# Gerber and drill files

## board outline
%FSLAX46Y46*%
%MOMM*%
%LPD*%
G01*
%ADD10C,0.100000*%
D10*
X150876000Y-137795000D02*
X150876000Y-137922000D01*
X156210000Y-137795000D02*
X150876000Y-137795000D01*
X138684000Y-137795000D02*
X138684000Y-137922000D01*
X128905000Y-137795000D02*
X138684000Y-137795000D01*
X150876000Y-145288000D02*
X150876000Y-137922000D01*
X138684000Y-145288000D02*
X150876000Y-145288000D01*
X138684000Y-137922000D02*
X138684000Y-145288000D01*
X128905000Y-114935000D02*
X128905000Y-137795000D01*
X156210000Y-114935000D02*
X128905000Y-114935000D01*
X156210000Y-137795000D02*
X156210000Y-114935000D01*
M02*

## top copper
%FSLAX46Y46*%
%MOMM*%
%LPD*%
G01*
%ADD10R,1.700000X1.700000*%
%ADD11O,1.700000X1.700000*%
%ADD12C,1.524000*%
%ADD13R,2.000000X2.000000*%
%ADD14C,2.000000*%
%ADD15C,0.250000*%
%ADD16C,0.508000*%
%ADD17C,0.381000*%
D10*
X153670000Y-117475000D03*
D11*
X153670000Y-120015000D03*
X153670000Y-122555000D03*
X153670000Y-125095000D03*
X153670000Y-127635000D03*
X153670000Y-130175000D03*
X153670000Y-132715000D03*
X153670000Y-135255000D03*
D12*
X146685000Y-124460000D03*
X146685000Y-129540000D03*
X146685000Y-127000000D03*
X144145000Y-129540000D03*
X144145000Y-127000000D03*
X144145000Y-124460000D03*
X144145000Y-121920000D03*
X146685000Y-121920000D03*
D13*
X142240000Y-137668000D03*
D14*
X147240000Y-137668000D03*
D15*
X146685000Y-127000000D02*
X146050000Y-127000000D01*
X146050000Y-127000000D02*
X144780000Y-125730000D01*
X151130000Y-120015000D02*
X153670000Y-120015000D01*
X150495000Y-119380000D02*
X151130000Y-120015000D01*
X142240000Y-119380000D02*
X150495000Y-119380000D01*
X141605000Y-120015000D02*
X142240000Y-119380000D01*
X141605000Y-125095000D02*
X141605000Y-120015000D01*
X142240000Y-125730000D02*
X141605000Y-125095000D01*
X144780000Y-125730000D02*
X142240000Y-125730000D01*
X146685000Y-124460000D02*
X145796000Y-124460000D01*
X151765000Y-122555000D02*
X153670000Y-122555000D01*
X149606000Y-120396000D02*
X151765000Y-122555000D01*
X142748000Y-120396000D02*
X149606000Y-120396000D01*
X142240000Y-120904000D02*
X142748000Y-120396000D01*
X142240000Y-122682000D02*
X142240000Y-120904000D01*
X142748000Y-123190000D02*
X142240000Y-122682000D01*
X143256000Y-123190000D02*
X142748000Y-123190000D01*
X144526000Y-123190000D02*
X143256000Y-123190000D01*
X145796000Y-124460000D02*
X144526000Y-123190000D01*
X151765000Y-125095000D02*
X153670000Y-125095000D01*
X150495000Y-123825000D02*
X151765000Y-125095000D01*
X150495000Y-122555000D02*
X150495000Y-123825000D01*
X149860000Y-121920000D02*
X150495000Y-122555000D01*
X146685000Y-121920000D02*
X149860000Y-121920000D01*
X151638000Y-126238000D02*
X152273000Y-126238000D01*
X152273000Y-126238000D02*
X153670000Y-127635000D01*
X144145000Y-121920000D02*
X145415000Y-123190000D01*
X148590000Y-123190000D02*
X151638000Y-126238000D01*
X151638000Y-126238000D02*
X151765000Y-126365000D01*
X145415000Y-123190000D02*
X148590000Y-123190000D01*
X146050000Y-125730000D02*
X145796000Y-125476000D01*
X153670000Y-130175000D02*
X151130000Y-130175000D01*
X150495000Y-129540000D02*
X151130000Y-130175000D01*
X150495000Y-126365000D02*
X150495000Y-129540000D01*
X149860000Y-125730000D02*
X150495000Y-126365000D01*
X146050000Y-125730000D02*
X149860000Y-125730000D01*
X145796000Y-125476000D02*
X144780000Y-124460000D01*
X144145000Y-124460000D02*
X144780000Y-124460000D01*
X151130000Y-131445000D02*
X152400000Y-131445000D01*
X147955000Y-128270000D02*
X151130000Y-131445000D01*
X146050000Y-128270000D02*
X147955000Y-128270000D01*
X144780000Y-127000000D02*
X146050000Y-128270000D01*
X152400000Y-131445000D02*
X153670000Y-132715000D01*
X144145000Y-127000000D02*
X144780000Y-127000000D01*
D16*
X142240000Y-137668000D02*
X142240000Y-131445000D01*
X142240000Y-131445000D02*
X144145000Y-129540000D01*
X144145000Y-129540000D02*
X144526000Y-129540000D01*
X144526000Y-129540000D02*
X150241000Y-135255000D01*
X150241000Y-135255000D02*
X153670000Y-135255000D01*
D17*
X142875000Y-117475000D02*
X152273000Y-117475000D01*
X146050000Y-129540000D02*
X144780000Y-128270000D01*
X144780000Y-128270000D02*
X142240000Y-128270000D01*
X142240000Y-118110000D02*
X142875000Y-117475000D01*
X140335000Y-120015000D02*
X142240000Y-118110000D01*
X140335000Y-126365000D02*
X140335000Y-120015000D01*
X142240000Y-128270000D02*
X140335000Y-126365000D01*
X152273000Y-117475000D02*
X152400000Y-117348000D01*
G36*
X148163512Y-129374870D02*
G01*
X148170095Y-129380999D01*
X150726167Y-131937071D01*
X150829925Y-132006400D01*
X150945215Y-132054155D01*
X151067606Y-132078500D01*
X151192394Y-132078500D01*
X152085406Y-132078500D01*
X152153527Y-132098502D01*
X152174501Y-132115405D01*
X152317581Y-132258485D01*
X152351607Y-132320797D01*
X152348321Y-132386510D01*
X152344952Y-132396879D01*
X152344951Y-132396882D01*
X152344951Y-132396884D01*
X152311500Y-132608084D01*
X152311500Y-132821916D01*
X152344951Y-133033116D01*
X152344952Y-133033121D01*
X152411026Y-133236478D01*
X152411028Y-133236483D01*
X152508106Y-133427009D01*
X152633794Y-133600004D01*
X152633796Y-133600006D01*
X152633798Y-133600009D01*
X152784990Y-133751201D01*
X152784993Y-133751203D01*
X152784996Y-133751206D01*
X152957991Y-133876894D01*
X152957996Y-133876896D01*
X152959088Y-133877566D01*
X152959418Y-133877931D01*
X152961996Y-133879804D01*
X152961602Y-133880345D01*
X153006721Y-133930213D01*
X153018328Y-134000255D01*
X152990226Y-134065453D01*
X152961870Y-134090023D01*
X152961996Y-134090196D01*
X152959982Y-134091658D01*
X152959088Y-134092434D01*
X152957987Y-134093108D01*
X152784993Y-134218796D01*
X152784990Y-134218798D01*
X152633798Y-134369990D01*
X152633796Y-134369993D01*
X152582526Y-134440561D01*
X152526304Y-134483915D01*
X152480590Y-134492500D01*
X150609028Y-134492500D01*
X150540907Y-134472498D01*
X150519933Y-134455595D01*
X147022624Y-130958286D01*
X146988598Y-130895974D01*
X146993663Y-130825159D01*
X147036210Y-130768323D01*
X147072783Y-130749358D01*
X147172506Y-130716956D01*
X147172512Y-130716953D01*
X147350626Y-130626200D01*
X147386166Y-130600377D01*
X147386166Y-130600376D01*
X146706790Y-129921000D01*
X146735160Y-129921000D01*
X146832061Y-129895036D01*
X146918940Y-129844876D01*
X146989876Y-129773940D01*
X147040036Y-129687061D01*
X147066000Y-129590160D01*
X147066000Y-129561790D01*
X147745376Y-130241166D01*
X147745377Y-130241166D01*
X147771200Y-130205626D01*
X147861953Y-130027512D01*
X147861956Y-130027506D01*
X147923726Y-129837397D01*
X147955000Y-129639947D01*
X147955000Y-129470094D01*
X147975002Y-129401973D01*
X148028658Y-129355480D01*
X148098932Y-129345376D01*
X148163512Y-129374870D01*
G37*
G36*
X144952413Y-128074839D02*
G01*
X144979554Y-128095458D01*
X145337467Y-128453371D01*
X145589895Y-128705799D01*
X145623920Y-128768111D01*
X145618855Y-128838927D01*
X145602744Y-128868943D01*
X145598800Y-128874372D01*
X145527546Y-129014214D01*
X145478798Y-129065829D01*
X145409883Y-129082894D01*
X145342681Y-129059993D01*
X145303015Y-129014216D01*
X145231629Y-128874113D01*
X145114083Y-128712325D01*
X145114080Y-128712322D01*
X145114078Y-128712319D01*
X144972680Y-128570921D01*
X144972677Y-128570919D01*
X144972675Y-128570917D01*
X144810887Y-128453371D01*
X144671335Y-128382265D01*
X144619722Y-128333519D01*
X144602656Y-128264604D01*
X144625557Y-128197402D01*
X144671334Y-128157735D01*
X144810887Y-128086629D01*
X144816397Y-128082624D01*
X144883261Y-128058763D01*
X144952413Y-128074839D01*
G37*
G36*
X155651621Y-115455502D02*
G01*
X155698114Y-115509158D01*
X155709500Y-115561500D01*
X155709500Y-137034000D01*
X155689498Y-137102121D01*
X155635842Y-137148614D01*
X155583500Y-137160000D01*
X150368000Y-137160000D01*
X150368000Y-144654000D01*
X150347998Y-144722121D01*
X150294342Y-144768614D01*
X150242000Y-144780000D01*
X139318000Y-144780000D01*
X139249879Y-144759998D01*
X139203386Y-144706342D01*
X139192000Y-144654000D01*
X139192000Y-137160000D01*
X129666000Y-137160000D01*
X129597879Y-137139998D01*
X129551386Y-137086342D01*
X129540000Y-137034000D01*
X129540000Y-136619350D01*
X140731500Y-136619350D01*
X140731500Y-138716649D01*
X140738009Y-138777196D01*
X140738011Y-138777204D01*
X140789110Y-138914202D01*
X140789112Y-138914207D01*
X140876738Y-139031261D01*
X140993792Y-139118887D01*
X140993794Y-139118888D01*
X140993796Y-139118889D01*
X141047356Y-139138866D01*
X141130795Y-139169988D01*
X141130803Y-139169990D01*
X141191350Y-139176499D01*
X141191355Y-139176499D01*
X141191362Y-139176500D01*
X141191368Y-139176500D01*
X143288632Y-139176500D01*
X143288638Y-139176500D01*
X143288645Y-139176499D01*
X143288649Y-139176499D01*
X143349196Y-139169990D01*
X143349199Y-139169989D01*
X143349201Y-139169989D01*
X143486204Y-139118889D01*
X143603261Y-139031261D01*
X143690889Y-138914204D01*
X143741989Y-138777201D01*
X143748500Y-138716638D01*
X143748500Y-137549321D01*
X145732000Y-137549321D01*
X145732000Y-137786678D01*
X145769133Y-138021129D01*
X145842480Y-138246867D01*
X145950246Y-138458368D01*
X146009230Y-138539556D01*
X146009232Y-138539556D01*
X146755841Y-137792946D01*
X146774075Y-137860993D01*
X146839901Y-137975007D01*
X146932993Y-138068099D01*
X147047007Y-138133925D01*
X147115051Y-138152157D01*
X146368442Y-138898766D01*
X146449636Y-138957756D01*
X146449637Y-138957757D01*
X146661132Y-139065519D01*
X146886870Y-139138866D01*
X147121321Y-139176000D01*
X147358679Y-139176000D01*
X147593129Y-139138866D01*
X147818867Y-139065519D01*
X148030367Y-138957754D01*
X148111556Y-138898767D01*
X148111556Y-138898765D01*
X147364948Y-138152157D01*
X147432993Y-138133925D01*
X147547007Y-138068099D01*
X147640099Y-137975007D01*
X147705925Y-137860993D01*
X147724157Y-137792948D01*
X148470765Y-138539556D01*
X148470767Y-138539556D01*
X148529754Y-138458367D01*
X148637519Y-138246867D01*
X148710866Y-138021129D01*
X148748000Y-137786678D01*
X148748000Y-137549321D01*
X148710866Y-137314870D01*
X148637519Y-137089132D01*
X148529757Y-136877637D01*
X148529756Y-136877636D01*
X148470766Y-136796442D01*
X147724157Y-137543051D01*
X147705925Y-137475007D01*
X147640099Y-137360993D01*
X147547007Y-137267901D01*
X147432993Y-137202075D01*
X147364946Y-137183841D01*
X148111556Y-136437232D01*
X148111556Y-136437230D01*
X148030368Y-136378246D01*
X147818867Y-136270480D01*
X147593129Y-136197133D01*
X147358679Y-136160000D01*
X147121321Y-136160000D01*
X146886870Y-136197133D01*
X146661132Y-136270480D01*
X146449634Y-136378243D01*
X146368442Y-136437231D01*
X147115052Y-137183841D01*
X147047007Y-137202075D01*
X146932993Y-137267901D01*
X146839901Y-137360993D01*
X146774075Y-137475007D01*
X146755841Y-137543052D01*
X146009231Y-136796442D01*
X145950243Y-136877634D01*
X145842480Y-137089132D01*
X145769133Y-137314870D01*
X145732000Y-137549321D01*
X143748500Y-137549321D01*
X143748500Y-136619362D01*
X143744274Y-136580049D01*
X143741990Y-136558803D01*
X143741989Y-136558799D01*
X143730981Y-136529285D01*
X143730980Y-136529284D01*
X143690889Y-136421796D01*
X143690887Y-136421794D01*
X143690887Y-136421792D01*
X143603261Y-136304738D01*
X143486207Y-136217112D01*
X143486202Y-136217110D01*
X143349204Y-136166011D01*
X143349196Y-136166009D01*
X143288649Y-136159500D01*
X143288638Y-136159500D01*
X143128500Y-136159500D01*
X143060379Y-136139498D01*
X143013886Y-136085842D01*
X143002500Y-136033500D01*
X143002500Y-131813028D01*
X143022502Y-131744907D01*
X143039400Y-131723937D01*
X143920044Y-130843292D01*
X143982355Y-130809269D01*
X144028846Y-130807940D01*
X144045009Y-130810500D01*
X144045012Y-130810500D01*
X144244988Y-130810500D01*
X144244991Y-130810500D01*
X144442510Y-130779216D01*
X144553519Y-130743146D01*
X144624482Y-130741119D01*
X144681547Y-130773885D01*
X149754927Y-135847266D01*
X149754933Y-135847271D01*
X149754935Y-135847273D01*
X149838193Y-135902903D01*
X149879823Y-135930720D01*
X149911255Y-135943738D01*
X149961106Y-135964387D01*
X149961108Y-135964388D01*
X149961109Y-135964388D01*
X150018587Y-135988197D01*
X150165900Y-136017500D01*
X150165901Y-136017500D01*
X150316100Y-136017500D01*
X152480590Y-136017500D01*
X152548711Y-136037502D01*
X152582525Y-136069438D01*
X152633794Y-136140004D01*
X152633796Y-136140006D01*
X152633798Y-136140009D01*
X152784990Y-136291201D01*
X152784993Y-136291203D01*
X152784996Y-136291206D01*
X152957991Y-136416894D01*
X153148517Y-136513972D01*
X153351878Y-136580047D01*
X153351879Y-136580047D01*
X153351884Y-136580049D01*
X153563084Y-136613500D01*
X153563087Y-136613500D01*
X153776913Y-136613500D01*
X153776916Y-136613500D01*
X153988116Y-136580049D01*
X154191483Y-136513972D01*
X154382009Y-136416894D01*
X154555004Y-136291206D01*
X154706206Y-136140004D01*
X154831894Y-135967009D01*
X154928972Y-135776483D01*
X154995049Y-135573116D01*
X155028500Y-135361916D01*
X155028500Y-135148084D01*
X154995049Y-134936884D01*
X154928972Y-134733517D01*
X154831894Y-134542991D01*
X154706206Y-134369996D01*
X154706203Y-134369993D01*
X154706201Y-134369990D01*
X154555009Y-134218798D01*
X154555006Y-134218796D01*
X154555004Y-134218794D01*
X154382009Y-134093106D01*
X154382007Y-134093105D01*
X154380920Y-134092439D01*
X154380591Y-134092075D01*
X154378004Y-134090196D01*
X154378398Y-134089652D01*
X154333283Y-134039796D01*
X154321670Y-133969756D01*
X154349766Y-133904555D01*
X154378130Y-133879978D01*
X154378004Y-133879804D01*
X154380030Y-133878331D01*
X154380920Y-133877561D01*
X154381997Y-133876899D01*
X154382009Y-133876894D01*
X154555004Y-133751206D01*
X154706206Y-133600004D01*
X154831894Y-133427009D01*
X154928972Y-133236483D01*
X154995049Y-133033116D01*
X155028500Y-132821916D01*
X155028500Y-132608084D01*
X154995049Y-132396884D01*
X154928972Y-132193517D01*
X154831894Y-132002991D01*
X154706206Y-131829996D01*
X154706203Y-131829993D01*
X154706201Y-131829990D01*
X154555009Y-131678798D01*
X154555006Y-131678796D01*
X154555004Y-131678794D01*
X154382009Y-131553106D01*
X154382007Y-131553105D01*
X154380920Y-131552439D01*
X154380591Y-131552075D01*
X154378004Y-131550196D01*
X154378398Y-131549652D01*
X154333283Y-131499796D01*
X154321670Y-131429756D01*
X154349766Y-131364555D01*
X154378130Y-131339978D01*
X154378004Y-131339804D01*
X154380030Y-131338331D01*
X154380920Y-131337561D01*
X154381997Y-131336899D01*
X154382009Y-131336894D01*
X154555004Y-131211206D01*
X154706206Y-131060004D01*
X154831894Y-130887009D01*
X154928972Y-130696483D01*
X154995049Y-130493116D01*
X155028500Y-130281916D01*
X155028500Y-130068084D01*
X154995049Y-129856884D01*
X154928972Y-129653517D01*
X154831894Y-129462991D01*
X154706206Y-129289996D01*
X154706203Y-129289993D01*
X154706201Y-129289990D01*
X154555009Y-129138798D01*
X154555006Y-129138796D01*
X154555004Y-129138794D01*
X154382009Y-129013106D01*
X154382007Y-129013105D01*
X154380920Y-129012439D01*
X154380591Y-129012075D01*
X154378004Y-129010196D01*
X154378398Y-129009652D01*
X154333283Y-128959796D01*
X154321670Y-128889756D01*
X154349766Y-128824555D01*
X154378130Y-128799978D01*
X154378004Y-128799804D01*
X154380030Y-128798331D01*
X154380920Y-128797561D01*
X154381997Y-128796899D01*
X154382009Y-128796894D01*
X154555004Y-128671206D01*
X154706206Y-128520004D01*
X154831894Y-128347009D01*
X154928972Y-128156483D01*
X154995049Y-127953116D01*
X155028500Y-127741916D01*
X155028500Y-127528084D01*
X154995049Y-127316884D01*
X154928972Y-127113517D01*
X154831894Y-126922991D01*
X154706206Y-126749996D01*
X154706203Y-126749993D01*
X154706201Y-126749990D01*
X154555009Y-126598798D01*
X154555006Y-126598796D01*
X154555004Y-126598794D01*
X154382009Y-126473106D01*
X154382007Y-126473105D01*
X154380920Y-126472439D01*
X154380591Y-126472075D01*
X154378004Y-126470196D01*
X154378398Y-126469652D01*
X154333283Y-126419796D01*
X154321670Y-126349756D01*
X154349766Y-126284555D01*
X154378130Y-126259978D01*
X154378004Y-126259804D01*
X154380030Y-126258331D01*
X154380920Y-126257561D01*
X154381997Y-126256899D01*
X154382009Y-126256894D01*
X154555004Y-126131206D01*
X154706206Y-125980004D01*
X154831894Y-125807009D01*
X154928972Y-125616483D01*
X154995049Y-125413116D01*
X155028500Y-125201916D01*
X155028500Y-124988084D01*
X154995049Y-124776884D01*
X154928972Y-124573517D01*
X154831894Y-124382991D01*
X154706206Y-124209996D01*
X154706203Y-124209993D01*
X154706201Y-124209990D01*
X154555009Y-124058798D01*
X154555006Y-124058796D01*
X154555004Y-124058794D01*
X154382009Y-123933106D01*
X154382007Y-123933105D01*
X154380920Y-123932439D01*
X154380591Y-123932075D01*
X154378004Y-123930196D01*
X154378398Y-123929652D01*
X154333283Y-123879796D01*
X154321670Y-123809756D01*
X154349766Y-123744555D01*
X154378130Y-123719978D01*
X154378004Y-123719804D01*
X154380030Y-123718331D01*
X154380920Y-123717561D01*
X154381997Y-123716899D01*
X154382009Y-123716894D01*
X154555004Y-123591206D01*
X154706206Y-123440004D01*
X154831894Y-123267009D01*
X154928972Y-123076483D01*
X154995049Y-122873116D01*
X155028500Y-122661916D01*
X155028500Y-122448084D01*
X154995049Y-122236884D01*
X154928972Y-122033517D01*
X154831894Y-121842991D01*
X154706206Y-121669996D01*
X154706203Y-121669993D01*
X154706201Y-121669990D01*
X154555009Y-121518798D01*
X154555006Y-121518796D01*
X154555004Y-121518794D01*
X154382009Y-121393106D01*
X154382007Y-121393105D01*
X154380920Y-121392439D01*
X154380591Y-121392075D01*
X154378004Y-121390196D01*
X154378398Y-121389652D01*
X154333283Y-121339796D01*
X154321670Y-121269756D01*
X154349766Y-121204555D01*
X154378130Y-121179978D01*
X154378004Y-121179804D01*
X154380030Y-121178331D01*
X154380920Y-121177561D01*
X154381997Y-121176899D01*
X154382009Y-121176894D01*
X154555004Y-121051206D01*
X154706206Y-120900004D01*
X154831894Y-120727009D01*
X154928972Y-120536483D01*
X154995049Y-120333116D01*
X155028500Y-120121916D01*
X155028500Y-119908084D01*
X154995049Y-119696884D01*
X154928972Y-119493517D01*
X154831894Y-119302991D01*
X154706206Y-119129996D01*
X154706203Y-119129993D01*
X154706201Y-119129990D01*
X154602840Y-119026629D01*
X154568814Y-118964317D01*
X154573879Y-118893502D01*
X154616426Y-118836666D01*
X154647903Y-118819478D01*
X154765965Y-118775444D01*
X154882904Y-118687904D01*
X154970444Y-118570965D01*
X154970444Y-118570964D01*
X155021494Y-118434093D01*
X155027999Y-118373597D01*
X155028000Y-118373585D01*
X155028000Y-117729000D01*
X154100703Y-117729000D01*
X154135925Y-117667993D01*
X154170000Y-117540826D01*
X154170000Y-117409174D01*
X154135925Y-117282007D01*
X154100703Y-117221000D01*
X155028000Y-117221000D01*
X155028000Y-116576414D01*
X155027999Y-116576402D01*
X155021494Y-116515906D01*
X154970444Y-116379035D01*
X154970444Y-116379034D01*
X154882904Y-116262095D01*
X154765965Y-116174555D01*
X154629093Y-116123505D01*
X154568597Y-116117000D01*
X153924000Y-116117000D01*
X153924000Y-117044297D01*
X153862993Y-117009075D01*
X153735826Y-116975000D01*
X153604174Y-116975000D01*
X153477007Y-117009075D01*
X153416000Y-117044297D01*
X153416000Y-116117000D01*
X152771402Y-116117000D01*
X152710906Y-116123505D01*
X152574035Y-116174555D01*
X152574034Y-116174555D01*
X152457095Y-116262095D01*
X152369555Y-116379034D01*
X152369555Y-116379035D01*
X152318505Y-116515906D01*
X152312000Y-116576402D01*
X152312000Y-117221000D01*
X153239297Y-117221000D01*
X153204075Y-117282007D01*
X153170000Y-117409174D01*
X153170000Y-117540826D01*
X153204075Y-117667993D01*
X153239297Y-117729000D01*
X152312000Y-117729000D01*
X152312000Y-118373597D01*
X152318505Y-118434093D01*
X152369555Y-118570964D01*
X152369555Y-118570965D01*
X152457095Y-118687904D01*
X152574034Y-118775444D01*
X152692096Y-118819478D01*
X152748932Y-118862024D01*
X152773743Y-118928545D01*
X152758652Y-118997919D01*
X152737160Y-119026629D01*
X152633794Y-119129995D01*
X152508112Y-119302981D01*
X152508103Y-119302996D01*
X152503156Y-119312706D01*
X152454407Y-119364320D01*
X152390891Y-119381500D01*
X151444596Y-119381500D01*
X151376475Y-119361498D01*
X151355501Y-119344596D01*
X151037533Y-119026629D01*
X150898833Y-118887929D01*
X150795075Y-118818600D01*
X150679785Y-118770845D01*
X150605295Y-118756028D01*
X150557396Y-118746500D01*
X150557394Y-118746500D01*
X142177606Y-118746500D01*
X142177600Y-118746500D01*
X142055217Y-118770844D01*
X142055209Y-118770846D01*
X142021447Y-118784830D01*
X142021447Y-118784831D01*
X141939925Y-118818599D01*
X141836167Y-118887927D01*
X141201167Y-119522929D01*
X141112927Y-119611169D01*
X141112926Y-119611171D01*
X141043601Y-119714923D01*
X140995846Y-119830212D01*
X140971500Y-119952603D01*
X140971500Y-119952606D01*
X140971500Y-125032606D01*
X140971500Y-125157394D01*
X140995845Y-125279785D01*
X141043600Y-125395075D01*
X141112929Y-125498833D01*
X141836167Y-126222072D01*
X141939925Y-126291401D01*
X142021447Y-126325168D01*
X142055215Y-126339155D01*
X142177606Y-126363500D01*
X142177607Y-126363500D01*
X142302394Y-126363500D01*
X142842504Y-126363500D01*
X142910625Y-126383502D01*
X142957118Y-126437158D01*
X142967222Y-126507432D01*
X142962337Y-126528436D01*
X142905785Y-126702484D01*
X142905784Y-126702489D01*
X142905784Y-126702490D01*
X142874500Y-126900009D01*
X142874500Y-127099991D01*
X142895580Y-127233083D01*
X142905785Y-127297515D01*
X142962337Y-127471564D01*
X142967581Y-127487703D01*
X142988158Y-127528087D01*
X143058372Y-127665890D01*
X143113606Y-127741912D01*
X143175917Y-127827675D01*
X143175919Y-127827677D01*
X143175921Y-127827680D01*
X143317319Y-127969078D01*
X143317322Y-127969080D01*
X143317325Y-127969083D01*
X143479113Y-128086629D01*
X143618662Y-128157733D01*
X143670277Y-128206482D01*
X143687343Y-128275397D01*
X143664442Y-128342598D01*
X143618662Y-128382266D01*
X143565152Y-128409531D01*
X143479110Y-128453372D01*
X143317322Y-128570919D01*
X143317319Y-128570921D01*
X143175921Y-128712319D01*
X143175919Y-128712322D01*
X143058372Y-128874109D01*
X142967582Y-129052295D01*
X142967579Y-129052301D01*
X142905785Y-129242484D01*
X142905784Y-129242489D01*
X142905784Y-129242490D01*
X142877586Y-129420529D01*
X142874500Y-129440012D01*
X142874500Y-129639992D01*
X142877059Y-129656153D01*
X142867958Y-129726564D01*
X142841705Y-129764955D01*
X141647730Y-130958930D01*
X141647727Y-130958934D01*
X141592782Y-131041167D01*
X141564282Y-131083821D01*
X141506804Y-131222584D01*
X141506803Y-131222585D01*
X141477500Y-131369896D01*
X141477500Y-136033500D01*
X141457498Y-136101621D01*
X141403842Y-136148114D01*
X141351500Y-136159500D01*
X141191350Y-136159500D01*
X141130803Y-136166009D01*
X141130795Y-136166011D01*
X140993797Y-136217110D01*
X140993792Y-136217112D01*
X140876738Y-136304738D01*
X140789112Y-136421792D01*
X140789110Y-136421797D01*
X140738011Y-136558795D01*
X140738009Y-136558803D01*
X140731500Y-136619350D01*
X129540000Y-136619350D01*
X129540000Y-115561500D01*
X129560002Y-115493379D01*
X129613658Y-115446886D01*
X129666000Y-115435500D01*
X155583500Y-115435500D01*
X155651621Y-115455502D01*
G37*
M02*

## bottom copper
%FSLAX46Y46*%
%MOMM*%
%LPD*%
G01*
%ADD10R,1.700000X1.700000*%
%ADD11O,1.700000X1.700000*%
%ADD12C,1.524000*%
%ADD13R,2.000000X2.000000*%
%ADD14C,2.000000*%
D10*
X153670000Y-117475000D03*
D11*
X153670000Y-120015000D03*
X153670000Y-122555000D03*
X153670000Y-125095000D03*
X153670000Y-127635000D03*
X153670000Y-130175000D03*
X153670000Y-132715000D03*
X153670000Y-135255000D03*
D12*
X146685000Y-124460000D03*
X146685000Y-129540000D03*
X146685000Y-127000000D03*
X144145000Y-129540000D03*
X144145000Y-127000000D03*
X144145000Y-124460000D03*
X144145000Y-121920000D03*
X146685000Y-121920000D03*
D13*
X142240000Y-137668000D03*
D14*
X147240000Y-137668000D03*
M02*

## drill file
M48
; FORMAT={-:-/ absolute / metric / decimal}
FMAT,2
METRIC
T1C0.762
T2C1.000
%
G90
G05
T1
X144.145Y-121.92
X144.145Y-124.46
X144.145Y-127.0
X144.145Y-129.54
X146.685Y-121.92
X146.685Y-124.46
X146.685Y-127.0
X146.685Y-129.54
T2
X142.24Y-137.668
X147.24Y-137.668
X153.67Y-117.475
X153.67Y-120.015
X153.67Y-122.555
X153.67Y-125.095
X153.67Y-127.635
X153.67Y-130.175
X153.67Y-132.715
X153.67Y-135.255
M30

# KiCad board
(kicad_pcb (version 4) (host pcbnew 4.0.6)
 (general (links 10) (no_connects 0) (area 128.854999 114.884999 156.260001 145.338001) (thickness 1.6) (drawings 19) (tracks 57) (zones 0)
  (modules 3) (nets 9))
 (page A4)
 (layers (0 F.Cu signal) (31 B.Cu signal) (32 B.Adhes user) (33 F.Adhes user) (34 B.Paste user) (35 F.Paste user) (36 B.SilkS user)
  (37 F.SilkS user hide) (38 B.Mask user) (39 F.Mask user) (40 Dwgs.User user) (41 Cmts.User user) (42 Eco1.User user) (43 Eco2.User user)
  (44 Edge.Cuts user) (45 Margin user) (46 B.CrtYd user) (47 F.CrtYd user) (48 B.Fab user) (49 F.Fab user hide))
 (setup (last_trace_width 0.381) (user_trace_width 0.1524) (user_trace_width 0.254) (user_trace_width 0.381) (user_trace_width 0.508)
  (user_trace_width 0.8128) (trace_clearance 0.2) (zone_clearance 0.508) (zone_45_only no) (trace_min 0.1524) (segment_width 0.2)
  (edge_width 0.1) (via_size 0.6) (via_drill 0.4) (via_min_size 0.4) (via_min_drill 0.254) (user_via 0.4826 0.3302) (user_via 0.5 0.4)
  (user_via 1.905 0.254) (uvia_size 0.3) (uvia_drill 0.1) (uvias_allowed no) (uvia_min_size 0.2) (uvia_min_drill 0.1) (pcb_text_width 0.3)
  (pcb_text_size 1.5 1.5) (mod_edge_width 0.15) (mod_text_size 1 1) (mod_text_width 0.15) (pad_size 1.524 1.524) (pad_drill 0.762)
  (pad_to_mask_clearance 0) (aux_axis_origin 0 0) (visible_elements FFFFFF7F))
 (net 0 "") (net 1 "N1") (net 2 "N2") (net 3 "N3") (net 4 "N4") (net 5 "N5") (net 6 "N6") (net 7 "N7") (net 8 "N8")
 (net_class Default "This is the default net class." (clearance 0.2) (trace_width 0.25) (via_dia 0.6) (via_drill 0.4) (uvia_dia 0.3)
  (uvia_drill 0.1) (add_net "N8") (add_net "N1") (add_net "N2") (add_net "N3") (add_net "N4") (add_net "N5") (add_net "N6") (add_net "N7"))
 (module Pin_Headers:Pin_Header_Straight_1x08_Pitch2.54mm (layer F.Cu) (at 153.67 117.475)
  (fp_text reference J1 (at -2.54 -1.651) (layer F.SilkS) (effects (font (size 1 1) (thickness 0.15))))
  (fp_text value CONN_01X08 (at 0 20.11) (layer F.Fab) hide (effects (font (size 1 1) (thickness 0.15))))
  (pad 1 thru_hole rect (at 0 0) (size 1.7 1.7) (drill 1) (layers *.Cu *.Mask) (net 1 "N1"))
  (pad 2 thru_hole oval (at 0 2.54) (size 1.7 1.7) (drill 1) (layers *.Cu *.Mask) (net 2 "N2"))
  (pad 3 thru_hole oval (at 0 5.08) (size 1.7 1.7) (drill 1) (layers *.Cu *.Mask) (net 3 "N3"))
  (pad 4 thru_hole oval (at 0 7.62) (size 1.7 1.7) (drill 1) (layers *.Cu *.Mask) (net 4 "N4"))
  (pad 5 thru_hole oval (at 0 10.16) (size 1.7 1.7) (drill 1) (layers *.Cu *.Mask) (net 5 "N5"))
  (pad 6 thru_hole oval (at 0 12.7) (size 1.7 1.7) (drill 1) (layers *.Cu *.Mask) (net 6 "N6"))
  (pad 7 thru_hole oval (at 0 15.24) (size 1.7 1.7) (drill 1) (layers *.Cu *.Mask) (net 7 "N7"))
  (pad 8 thru_hole oval (at 0 17.78) (size 1.7 1.7) (drill 1) (layers *.Cu *.Mask) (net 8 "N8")))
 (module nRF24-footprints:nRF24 (layer F.Cu) (at 144.145 127)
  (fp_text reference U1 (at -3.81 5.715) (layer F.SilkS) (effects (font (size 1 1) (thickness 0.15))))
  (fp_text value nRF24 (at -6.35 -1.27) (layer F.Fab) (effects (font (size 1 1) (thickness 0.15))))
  (pad 2 thru_hole circle (at 2.54 -2.54) (size 1.524 1.524) (drill 0.762) (layers *.Cu *.Mask) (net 3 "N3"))
  (pad 0 thru_hole circle (at 2.54 2.54) (size 1.524 1.524) (drill 0.762) (layers *.Cu *.Mask) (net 1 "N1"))
  (pad 1 thru_hole circle (at 2.54 0) (size 1.524 1.524) (drill 0.762) (layers *.Cu *.Mask) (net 2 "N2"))
  (pad 7 thru_hole circle (at 0 2.54) (size 1.524 1.524) (drill 0.762) (layers *.Cu *.Mask) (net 8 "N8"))
  (pad 6 thru_hole circle (at 0 0) (size 1.524 1.524) (drill 0.762) (layers *.Cu *.Mask) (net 7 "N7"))
  (pad 5 thru_hole circle (at 0 -2.54) (size 1.524 1.524) (drill 0.762) (layers *.Cu *.Mask) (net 6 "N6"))
  (pad 4 thru_hole circle (at 0 -5.08) (size 1.524 1.524) (drill 0.762) (layers *.Cu *.Mask) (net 5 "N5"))
  (pad 3 thru_hole circle (at 2.54 -5.08) (size 1.524 1.524) (drill 0.762) (layers *.Cu *.Mask) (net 4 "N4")))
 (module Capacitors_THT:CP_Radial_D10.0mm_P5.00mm (layer F.Cu) (at 142.24 137.668)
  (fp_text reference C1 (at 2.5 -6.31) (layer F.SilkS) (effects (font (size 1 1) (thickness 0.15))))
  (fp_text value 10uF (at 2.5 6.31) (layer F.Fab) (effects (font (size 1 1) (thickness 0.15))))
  (pad 1 thru_hole rect (at 0 0) (size 2 2) (drill 1) (layers *.Cu *.Mask) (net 8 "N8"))
  (pad 2 thru_hole circle (at 5 0) (size 2 2) (drill 1) (layers *.Cu *.Mask) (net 1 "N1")))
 (gr_line (start 150.876 137.795) (end 150.876 137.922) (angle 90) (layer Edge.Cuts) (width 0.1))
 (gr_line (start 156.21 137.795) (end 150.876 137.795) (angle 90) (layer Edge.Cuts) (width 0.1))
 (gr_line (start 138.684 137.795) (end 138.684 137.922) (angle 90) (layer Edge.Cuts) (width 0.1))
 (gr_line (start 128.905 137.795) (end 138.684 137.795) (angle 90) (layer Edge.Cuts) (width 0.1))
 (gr_line (start 150.876 145.288) (end 150.876 137.922) (angle 90) (layer Edge.Cuts) (width 0.1))
 (gr_line (start 138.684 145.288) (end 150.876 145.288) (angle 90) (layer Edge.Cuts) (width 0.1))
 (gr_line (start 138.684 137.922) (end 138.684 145.288) (angle 90) (layer Edge.Cuts) (width 0.1))
 (gr_line (start 128.905 114.935) (end 128.905 137.795) (angle 90) (layer Edge.Cuts) (width 0.1))
 (gr_line (start 156.21 114.935) (end 128.905 114.935) (angle 90) (layer Edge.Cuts) (width 0.1))
 (gr_line (start 156.21 137.795) (end 156.21 114.935) (angle 90) (layer Edge.Cuts) (width 0.1))
 (segment (start 146.685 127) (end 146.05 127) (width 0.25) (layer F.Cu) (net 2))
 (segment (start 146.05 127) (end 144.78 125.73) (width 0.25) (layer F.Cu) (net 2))
 (segment (start 151.13 120.015) (end 153.67 120.015) (width 0.25) (layer F.Cu) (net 2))
 (segment (start 150.495 119.38) (end 151.13 120.015) (width 0.25) (layer F.Cu) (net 2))
 (segment (start 142.24 119.38) (end 150.495 119.38) (width 0.25) (layer F.Cu) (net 2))
 (segment (start 141.605 120.015) (end 142.24 119.38) (width 0.25) (layer F.Cu) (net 2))
 (segment (start 141.605 125.095) (end 141.605 120.015) (width 0.25) (layer F.Cu) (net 2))
 (segment (start 142.24 125.73) (end 141.605 125.095) (width 0.25) (layer F.Cu) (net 2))
 (segment (start 144.78 125.73) (end 142.24 125.73) (width 0.25) (layer F.Cu) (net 2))
 (segment (start 146.685 124.46) (end 145.796 124.46) (width 0.25) (layer F.Cu) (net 3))
 (segment (start 151.765 122.555) (end 153.67 122.555) (width 0.25) (layer F.Cu) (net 3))
 (segment (start 149.606 120.396) (end 151.765 122.555) (width 0.25) (layer F.Cu) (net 3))
 (segment (start 142.748 120.396) (end 149.606 120.396) (width 0.25) (layer F.Cu) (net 3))
 (segment (start 142.24 120.904) (end 142.748 120.396) (width 0.25) (layer F.Cu) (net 3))
 (segment (start 142.24 122.682) (end 142.24 120.904) (width 0.25) (layer F.Cu) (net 3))
 (segment (start 142.748 123.19) (end 142.24 122.682) (width 0.25) (layer F.Cu) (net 3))
 (segment (start 143.256 123.19) (end 142.748 123.19) (width 0.25) (layer F.Cu) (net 3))
 (segment (start 144.526 123.19) (end 143.256 123.19) (width 0.25) (layer F.Cu) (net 3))
 (segment (start 145.796 124.46) (end 144.526 123.19) (width 0.25) (layer F.Cu) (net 3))
 (segment (start 151.765 125.095) (end 153.67 125.095) (width 0.25) (layer F.Cu) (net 4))
 (segment (start 150.495 123.825) (end 151.765 125.095) (width 0.25) (layer F.Cu) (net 4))
 (segment (start 150.495 122.555) (end 150.495 123.825) (width 0.25) (layer F.Cu) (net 4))
 (segment (start 149.86 121.92) (end 150.495 122.555) (width 0.25) (layer F.Cu) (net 4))
 (segment (start 146.685 121.92) (end 149.86 121.92) (width 0.25) (layer F.Cu) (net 4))
 (segment (start 151.638 126.238) (end 152.273 126.238) (width 0.25) (layer F.Cu) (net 5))
 (segment (start 152.273 126.238) (end 153.67 127.635) (width 0.25) (layer F.Cu) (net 5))
 (segment (start 144.145 121.92) (end 145.415 123.19) (width 0.25) (layer F.Cu) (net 5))
 (segment (start 148.59 123.19) (end 151.638 126.238) (width 0.25) (layer F.Cu) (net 5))
 (segment (start 151.638 126.238) (end 151.765 126.365) (width 0.25) (layer F.Cu) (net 5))
 (segment (start 145.415 123.19) (end 148.59 123.19) (width 0.25) (layer F.Cu) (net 5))
 (segment (start 146.05 125.73) (end 145.796 125.476) (width 0.25) (layer F.Cu) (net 6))
 (segment (start 153.67 130.175) (end 151.13 130.175) (width 0.25) (layer F.Cu) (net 6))
 (segment (start 150.495 129.54) (end 151.13 130.175) (width 0.25) (layer F.Cu) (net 6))
 (segment (start 150.495 126.365) (end 150.495 129.54) (width 0.25) (layer F.Cu) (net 6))
 (segment (start 149.86 125.73) (end 150.495 126.365) (width 0.25) (layer F.Cu) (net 6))
 (segment (start 146.05 125.73) (end 149.86 125.73) (width 0.25) (layer F.Cu) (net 6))
 (segment (start 145.796 125.476) (end 144.78 124.46) (width 0.25) (layer F.Cu) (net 6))
 (segment (start 144.145 124.46) (end 144.78 124.46) (width 0.25) (layer F.Cu) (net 6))
 (segment (start 151.13 131.445) (end 152.4 131.445) (width 0.25) (layer F.Cu) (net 7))
 (segment (start 147.955 128.27) (end 151.13 131.445) (width 0.25) (layer F.Cu) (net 7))
 (segment (start 146.05 128.27) (end 147.955 128.27) (width 0.25) (layer F.Cu) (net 7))
 (segment (start 144.78 127) (end 146.05 128.27) (width 0.25) (layer F.Cu) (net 7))
 (segment (start 152.4 131.445) (end 153.67 132.715) (width 0.25) (layer F.Cu) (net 7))
 (segment (start 144.145 127) (end 144.78 127) (width 0.25) (layer F.Cu) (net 7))
 (segment (start 142.24 137.668) (end 142.24 131.445) (width 0.508) (layer F.Cu) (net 8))
 (segment (start 142.24 131.445) (end 144.145 129.54) (width 0.508) (layer F.Cu) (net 8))
 (segment (start 144.145 129.54) (end 144.526 129.54) (width 0.508) (layer F.Cu) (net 8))
 (segment (start 144.526 129.54) (end 150.241 135.255) (width 0.508) (layer F.Cu) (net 8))
 (segment (start 150.241 135.255) (end 153.67 135.255) (width 0.508) (layer F.Cu) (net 8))
 (segment (start 142.875 117.475) (end 152.273 117.475) (width 0.381) (layer F.Cu) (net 1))
 (segment (start 146.05 129.54) (end 144.78 128.27) (width 0.381) (layer F.Cu) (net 1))
 (segment (start 144.78 128.27) (end 142.24 128.27) (width 0.381) (layer F.Cu) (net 1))
 (segment (start 142.24 118.11) (end 142.875 117.475) (width 0.381) (layer F.Cu) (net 1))
 (segment (start 140.335 120.015) (end 142.24 118.11) (width 0.381) (layer F.Cu) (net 1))
 (segment (start 140.335 126.365) (end 140.335 120.015) (width 0.381) (layer F.Cu) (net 1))
 (segment (start 142.24 128.27) (end 140.335 126.365) (width 0.381) (layer F.Cu) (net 1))
 (segment (start 152.273 117.475) (end 152.4 117.348) (width 0.381) (layer F.Cu) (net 1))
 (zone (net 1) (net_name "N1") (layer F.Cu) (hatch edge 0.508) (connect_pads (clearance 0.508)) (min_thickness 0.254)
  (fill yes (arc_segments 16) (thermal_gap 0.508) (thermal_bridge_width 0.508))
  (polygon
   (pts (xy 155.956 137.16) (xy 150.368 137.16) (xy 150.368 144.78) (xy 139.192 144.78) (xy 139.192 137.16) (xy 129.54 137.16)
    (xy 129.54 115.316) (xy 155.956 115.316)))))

